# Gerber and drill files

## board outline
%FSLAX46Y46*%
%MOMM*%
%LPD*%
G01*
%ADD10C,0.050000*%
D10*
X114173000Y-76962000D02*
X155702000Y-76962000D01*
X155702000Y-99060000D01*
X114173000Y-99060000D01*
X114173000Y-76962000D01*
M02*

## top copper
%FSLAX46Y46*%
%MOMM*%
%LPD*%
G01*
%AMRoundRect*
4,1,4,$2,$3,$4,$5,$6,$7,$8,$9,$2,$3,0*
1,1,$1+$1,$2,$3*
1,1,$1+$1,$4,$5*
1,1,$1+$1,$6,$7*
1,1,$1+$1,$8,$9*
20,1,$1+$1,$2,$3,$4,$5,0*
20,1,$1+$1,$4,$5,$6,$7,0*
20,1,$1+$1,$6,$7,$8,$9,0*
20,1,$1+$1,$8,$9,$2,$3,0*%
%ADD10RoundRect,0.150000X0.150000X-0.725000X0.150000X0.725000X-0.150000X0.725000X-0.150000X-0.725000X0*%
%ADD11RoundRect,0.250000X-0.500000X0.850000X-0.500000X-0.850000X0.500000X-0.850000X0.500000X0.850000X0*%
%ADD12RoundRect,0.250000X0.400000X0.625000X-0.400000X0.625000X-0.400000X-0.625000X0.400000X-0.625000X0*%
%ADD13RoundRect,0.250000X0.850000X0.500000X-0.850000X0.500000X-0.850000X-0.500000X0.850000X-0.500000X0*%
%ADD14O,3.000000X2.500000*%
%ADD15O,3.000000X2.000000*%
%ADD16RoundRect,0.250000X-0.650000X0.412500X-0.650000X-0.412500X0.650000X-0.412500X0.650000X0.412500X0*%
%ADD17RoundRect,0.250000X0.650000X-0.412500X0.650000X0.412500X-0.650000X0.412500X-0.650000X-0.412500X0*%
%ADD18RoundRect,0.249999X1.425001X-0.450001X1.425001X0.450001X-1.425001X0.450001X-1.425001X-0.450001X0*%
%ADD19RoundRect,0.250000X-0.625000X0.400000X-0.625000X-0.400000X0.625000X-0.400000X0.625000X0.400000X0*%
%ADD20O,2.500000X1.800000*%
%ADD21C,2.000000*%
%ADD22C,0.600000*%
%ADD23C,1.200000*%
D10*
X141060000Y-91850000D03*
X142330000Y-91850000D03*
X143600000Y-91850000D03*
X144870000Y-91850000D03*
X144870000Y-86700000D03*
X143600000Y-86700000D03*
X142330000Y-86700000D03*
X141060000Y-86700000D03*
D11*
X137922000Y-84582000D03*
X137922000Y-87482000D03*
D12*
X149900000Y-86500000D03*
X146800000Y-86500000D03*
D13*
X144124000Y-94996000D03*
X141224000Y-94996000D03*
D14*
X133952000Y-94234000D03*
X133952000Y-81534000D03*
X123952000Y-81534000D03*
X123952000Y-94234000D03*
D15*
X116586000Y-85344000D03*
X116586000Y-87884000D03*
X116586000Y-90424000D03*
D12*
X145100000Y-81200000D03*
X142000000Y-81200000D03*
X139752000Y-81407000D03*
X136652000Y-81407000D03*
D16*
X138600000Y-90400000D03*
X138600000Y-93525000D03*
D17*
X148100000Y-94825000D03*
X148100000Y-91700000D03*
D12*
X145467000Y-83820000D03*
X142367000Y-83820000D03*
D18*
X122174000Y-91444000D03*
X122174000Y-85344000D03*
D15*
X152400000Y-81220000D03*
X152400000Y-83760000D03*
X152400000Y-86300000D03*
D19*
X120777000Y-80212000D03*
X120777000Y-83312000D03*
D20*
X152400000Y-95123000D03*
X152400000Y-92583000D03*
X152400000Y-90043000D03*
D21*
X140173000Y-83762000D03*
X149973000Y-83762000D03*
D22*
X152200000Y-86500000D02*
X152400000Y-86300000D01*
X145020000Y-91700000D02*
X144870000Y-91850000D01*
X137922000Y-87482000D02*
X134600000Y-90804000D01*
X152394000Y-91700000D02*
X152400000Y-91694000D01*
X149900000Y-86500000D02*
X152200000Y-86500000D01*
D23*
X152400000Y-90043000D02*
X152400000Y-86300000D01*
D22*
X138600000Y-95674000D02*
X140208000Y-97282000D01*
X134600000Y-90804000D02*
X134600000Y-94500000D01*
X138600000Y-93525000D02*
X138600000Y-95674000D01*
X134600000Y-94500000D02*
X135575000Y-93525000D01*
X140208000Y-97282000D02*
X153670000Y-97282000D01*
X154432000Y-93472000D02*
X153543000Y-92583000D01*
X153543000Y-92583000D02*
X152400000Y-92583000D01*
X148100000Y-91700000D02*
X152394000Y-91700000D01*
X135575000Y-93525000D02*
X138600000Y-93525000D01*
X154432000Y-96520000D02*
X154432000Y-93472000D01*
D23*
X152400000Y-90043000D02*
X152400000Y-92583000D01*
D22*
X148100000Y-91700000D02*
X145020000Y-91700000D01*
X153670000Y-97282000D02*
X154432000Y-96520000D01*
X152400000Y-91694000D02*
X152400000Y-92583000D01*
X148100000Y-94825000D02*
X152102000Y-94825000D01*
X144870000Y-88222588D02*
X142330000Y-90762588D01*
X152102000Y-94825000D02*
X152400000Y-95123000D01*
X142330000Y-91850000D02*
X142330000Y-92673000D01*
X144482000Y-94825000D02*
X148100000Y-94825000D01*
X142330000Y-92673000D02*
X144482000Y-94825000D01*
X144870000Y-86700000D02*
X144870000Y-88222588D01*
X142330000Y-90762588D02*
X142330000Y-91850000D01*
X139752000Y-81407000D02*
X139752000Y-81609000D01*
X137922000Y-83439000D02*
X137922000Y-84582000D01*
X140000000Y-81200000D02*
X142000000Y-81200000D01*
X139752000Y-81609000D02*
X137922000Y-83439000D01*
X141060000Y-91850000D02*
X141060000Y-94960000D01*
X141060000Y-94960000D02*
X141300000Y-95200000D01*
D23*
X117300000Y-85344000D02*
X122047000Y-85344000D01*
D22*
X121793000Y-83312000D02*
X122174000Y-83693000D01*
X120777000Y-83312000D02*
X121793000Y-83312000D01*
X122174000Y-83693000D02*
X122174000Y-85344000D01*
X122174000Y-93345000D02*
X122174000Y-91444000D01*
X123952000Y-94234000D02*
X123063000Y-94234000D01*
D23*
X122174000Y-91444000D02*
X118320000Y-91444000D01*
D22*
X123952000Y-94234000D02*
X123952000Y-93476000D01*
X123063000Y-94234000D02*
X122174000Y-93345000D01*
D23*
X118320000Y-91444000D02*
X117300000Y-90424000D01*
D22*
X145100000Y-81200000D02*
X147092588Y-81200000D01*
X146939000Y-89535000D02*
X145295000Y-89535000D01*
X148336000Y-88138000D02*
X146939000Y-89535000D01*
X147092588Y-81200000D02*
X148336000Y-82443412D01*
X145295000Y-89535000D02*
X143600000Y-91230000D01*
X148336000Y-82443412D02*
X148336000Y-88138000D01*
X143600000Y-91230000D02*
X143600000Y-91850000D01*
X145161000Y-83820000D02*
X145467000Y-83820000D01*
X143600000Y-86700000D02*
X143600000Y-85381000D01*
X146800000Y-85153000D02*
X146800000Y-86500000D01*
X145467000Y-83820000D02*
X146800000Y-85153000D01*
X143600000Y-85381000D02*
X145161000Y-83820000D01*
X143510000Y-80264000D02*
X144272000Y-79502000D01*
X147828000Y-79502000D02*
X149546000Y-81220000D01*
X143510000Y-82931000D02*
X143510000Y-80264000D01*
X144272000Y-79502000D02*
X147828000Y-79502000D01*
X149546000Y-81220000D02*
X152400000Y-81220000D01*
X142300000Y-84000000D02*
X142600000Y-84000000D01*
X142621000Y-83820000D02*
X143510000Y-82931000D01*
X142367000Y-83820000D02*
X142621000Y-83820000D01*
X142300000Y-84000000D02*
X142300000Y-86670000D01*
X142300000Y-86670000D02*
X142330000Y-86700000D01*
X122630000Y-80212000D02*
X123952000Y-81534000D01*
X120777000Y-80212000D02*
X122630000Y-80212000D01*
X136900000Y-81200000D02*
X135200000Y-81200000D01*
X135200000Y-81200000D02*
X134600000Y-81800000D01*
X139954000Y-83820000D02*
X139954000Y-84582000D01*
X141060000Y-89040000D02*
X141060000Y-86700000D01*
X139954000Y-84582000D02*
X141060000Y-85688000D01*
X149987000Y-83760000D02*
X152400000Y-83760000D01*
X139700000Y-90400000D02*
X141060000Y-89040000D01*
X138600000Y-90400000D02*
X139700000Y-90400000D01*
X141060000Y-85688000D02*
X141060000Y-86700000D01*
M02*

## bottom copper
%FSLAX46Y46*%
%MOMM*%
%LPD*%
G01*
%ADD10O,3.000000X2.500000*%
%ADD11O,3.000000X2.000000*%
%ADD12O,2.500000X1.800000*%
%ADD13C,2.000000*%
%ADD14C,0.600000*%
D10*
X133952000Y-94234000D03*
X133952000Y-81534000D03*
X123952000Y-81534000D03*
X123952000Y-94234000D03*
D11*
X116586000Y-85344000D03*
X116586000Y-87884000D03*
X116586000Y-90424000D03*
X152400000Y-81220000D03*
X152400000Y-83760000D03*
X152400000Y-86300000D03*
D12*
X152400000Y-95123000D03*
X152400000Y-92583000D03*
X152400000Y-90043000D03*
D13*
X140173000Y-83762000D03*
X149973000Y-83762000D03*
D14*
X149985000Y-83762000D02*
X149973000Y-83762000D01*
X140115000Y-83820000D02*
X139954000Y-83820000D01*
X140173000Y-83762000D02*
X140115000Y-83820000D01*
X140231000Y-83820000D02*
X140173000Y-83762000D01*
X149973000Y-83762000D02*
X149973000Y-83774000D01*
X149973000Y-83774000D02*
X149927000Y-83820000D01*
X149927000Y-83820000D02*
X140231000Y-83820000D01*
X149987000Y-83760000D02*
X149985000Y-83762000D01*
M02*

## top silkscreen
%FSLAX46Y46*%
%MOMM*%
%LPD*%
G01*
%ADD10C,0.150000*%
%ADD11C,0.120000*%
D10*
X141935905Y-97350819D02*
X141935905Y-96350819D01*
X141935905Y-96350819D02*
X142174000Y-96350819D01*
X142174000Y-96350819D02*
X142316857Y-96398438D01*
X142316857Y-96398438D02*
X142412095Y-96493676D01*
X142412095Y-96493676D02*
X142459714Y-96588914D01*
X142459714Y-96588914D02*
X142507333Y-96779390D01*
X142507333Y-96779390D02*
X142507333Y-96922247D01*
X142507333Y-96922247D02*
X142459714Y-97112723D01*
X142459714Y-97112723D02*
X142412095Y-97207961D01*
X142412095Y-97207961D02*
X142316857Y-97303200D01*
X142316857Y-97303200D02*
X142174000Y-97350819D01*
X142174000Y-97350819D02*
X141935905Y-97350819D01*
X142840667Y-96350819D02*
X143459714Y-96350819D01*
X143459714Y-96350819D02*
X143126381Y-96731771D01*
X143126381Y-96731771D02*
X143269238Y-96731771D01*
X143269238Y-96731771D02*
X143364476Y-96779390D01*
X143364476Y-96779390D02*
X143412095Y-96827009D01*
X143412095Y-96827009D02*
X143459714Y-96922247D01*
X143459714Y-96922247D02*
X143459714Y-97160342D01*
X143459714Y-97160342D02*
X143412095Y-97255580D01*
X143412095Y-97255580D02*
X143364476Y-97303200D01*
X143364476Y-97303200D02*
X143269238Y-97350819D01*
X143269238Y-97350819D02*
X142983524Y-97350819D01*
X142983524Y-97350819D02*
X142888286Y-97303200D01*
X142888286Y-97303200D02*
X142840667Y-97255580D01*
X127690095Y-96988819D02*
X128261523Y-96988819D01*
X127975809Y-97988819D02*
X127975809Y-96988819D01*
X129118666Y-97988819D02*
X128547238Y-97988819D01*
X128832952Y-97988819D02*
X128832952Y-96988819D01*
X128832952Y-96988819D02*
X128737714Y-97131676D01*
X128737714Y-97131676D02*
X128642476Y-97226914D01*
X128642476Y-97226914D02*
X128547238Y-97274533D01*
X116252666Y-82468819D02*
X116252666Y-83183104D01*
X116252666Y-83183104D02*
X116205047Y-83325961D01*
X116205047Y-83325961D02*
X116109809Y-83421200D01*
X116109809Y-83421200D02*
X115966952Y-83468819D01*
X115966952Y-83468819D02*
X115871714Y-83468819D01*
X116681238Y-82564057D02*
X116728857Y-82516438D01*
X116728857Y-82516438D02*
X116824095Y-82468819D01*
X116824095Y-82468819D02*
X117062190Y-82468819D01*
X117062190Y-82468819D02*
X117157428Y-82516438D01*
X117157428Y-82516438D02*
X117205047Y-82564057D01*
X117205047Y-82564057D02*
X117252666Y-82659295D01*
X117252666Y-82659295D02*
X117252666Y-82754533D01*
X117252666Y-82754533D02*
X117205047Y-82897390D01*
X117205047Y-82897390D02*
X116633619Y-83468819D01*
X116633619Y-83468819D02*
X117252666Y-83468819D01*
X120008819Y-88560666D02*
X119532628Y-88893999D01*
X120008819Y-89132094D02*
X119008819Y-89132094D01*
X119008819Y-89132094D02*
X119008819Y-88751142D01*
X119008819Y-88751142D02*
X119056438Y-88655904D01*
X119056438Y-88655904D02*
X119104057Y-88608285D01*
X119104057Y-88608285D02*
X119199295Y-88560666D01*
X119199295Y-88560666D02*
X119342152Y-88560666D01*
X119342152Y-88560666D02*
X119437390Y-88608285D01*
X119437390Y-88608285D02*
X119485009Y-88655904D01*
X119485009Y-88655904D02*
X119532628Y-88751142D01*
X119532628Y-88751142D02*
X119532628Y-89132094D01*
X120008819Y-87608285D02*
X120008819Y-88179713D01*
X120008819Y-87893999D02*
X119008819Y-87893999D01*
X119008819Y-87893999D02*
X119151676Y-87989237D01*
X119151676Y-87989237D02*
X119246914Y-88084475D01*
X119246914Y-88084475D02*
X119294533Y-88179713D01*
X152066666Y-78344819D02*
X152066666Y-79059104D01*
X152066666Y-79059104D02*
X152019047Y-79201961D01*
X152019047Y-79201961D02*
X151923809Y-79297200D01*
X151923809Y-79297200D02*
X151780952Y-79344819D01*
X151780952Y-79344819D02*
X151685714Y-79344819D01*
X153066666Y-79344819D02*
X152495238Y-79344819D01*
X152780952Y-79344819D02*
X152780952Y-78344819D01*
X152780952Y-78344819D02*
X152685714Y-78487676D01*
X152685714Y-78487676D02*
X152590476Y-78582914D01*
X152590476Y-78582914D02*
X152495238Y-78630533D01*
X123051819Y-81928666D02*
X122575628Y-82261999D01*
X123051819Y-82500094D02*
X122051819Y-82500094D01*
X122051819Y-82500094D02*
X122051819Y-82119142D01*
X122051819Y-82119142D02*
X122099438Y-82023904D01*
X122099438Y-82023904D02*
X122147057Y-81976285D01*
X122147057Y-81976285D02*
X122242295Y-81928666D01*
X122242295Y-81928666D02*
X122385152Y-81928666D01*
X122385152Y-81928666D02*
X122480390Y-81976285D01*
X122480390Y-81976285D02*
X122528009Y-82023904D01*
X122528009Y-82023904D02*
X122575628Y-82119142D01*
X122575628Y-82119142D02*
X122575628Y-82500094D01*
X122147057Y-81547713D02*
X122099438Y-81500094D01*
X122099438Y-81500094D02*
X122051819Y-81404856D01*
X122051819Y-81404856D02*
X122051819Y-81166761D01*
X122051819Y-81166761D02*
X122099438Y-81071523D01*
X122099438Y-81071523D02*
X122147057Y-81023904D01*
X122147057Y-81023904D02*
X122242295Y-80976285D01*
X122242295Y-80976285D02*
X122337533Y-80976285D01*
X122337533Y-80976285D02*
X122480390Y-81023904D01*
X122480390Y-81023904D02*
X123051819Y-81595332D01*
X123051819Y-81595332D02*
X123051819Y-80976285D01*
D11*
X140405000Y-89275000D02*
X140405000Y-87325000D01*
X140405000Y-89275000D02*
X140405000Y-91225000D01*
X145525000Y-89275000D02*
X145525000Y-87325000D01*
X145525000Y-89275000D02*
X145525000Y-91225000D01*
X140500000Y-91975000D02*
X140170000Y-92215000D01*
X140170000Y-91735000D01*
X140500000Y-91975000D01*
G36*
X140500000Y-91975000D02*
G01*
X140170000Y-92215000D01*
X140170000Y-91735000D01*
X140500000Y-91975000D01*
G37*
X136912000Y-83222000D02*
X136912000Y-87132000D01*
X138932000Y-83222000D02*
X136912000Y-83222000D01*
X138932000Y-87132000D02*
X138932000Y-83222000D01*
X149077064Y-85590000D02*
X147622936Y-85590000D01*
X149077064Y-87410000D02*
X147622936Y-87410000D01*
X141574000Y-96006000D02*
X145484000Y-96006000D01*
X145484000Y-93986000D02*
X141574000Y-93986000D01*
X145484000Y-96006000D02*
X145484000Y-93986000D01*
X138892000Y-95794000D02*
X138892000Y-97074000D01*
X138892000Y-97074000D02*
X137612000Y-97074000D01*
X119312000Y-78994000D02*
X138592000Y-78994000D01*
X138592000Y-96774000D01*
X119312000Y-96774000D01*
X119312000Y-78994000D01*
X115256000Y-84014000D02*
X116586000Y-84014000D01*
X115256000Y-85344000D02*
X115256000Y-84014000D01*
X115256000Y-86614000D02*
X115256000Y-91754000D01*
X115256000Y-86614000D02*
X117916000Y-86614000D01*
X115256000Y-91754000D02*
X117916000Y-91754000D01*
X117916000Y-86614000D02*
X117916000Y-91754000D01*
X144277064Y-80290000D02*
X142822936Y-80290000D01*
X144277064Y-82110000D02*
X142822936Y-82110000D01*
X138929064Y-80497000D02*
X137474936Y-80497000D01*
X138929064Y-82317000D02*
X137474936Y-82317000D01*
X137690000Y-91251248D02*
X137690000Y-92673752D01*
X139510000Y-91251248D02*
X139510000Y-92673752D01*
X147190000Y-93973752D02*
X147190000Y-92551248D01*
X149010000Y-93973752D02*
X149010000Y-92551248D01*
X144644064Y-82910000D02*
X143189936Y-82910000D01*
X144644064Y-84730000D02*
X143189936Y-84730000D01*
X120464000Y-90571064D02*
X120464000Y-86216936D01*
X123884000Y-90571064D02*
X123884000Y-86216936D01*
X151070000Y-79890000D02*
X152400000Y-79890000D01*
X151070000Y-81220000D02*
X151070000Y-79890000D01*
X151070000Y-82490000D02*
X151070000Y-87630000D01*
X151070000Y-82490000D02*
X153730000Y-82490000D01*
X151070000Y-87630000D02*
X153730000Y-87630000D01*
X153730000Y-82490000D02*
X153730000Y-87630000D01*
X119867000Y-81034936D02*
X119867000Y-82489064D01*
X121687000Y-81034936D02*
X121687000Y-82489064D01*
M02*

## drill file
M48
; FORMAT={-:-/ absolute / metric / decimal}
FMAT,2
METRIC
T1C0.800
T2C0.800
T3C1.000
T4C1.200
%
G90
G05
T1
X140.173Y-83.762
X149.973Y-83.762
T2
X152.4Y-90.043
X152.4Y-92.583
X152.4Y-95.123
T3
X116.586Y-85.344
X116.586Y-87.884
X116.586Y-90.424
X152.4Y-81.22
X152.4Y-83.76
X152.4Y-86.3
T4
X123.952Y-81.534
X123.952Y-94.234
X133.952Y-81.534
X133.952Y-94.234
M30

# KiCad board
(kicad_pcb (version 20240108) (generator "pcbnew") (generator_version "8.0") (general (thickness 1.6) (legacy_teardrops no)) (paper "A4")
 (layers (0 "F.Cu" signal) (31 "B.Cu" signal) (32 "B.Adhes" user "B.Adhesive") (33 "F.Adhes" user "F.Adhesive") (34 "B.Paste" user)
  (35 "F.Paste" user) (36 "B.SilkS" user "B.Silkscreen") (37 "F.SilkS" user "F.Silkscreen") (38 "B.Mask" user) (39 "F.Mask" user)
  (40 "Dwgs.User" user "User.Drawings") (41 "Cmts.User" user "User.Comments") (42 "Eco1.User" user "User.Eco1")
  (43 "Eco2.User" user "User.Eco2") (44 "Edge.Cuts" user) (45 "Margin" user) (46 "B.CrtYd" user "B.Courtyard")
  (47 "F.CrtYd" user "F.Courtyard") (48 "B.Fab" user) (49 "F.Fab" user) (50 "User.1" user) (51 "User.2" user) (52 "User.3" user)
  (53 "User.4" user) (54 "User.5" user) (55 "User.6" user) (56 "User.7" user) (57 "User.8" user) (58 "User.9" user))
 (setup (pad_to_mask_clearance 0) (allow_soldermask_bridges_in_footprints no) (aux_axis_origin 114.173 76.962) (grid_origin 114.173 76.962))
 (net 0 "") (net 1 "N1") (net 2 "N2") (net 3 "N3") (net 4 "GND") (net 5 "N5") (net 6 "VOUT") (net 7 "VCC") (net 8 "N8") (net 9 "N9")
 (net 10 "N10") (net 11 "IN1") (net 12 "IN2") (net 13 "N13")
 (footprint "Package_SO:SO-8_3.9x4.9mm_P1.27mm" (layer "F.Cu") (at 142.965 89.275 90)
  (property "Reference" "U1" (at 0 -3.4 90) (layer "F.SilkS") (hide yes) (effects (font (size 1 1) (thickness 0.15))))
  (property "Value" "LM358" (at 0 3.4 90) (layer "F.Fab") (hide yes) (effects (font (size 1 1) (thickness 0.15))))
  (fp_line (start 0 -2.56) (end 1.95 -2.56) (stroke (width 0.12) (type solid)) (layer "F.SilkS"))
  (fp_line (start 0 -2.56) (end -1.95 -2.56) (stroke (width 0.12) (type solid)) (layer "F.SilkS"))
  (fp_line (start 0 2.56) (end 1.95 2.56) (stroke (width 0.12) (type solid)) (layer "F.SilkS"))
  (fp_line (start 0 2.56) (end -1.95 2.56) (stroke (width 0.12) (type solid)) (layer "F.SilkS"))
  (fp_poly
   (pts (xy -2.7 -2.465) (xy -2.94 -2.795) (xy -2.46 -2.795) (xy -2.7 -2.465)) (stroke (width 0.12) (type solid)) (fill solid)
   (layer "F.SilkS"))
  (pad "1" smd roundrect (at -2.575 -1.905 90) (size 1.75 0.6) (layers "F.Cu" "F.Paste" "F.Mask") (roundrect_rratio 0.25) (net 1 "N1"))
  (pad "2" smd roundrect (at -2.575 -0.635 90) (size 1.75 0.6) (layers "F.Cu" "F.Paste" "F.Mask") (roundrect_rratio 0.25) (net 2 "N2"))
  (pad "3" smd roundrect (at -2.575 0.635 90) (size 1.75 0.6) (layers "F.Cu" "F.Paste" "F.Mask") (roundrect_rratio 0.25) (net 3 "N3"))
  (pad "4" smd roundrect (at -2.575 1.905 90) (size 1.75 0.6) (layers "F.Cu" "F.Paste" "F.Mask") (roundrect_rratio 0.25) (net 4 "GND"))
  (pad "5" smd roundrect (at 2.575 1.905 90) (size 1.75 0.6) (layers "F.Cu" "F.Paste" "F.Mask") (roundrect_rratio 0.25) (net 2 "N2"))
  (pad "6" smd roundrect (at 2.575 0.635 90) (size 1.75 0.6) (layers "F.Cu" "F.Paste" "F.Mask") (roundrect_rratio 0.25) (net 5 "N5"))
  (pad "7" smd roundrect (at 2.575 -0.635 90) (size 1.75 0.6) (layers "F.Cu" "F.Paste" "F.Mask") (roundrect_rratio 0.25) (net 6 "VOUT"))
  (pad "8" smd roundrect (at 2.575 -1.905 90) (size 1.75 0.6) (layers "F.Cu" "F.Paste" "F.Mask") (roundrect_rratio 0.25) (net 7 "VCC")))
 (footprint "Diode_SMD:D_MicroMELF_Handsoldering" (layer "F.Cu") (at 137.922 86.032 -90)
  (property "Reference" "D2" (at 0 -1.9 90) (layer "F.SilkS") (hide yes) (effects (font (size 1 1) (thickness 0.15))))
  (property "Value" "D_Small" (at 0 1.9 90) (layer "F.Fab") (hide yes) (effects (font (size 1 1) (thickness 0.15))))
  (fp_line (start -2.81 1.01) (end 1.1 1.01) (stroke (width 0.12) (type solid)) (layer "F.SilkS"))
  (fp_line (start -2.81 -1.01) (end -2.81 1.01) (stroke (width 0.12) (type solid)) (layer "F.SilkS"))
  (fp_line (start 1.1 -1.01) (end -2.81 -1.01) (stroke (width 0.12) (type solid)) (layer "F.SilkS"))
  (pad "1" smd roundrect (at -1.45 0 270) (size 2.2 1.5) (layers "F.Cu" "F.Paste" "F.Mask") (roundrect_rratio 0.1666666667) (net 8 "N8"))
  (pad "2" smd roundrect (at 1.45 0 270) (size 2.2 1.5) (layers "F.Cu" "F.Paste" "F.Mask") (roundrect_rratio 0.1666666667) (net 4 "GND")))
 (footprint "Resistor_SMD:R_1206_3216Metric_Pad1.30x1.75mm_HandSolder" (layer "F.Cu") (at 148.35 86.5 180)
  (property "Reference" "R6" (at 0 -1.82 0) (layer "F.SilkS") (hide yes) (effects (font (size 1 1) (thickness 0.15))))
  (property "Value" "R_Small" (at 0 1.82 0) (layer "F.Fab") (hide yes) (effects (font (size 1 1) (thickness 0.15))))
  (fp_line (start -0.727064 0.91) (end 0.727064 0.91) (stroke (width 0.12) (type solid)) (layer "F.SilkS"))
  (fp_line (start -0.727064 -0.91) (end 0.727064 -0.91) (stroke (width 0.12) (type solid)) (layer "F.SilkS"))
  (pad "1" smd roundrect (at -1.55 0 180) (size 1.3 1.75) (layers "F.Cu" "F.Paste" "F.Mask") (roundrect_rratio 0.192308) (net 4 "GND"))
  (pad "2" smd roundrect (at 1.55 0 180) (size 1.3 1.75) (layers "F.Cu" "F.Paste" "F.Mask") (roundrect_rratio 0.192308) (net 5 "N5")))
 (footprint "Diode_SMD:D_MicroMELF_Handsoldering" (layer "F.Cu") (at 142.674 94.996 180)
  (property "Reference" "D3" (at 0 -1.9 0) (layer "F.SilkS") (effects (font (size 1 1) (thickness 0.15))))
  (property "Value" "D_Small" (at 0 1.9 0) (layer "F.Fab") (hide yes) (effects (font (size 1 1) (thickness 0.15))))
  (fp_line (start 1.1 -1.01) (end -2.81 -1.01) (stroke (width 0.12) (type solid)) (layer "F.SilkS"))
  (fp_line (start -2.81 1.01) (end 1.1 1.01) (stroke (width 0.12) (type solid)) (layer "F.SilkS"))
  (fp_line (start -2.81 -1.01) (end -2.81 1.01) (stroke (width 0.12) (type solid)) (layer "F.SilkS"))
  (pad "1" smd roundrect (at -1.45 0 180) (size 2.2 1.5) (layers "F.Cu" "F.Paste" "F.Mask") (roundrect_rratio 0.1666666667) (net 2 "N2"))
  (pad "2" smd roundrect (at 1.45 0 180) (size 2.2 1.5) (layers "F.Cu" "F.Paste" "F.Mask") (roundrect_rratio 0.1666666667) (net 1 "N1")))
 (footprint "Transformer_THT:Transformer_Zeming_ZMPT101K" (layer "F.Cu") (at 133.952 94.234 180)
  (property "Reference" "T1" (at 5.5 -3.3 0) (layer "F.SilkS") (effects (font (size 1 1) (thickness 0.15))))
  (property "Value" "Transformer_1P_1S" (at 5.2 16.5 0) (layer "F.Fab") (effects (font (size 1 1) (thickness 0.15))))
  (fp_line (start -4.94 -1.56) (end -4.94 -2.84) (stroke (width 0.12) (type default)) (layer "F.SilkS"))
  (fp_line (start -4.94 -2.84) (end -3.66 -2.84) (stroke (width 0.12) (type default)) (layer "F.SilkS"))
  (fp_rect (start -4.64 -2.54) (end 14.64 15.24) (stroke (width 0.12) (type default)) (fill none) (layer "F.SilkS"))
  (pad "1" thru_hole oval (at 0 0 180) (size 3 2.5) (drill 1.2) (layers "*.Cu" "*.Mask") (remove_unused_layers no) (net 4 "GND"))
  (pad "2" thru_hole oval (at 0 12.7 180) (size 3 2.5) (drill 1.2) (layers "*.Cu" "*.Mask") (remove_unused_layers no) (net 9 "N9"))
  (pad "3" thru_hole oval (at 10 12.7 180) (size 3 2.5) (drill 1.2) (layers "*.Cu" "*.Mask") (remove_unused_layers no) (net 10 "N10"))
  (pad "4" thru_hole oval (at 10 0 180) (size 3 2.5) (drill 1.2) (layers "*.Cu" "*.Mask") (remove_unused_layers no) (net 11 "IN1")))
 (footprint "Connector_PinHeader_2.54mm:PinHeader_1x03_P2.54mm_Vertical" (layer "F.Cu") (at 116.586 85.344)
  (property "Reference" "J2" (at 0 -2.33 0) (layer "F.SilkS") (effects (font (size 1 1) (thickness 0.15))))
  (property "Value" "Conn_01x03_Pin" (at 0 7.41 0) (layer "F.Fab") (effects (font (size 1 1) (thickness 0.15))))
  (fp_line (start -1.33 -1.33) (end 0 -1.33) (stroke (width 0.12) (type solid)) (layer "F.SilkS"))
  (fp_line (start -1.33 0) (end -1.33 -1.33) (stroke (width 0.12) (type solid)) (layer "F.SilkS"))
  (fp_line (start -1.33 1.27) (end -1.33 6.41) (stroke (width 0.12) (type solid)) (layer "F.SilkS"))
  (fp_line (start -1.33 1.27) (end 1.33 1.27) (stroke (width 0.12) (type solid)) (layer "F.SilkS"))
  (fp_line (start -1.33 6.41) (end 1.33 6.41) (stroke (width 0.12) (type solid)) (layer "F.SilkS"))
  (fp_line (start 1.33 1.27) (end 1.33 6.41) (stroke (width 0.12) (type solid)) (layer "F.SilkS"))
  (pad "1" thru_hole oval (at 0 0) (size 3 2) (drill 1) (layers "*.Cu" "*.Mask") (remove_unused_layers no) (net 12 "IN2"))
  (pad "2" thru_hole oval (at 0 2.54) (size 3 2) (drill 1) (layers "*.Cu" "*.Mask") (remove_unused_layers no) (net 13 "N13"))
  (pad "3" thru_hole oval (at 0 5.08) (size 3 2) (drill 1) (layers "*.Cu" "*.Mask") (remove_unused_layers no) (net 11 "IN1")))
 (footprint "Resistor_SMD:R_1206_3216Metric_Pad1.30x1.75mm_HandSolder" (layer "F.Cu") (at 143.55 81.2 180)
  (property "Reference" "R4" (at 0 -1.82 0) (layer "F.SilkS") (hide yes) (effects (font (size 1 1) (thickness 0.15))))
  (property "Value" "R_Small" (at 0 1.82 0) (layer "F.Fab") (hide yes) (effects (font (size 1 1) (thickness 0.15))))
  (fp_line (start -0.727064 0.91) (end 0.727064 0.91) (stroke (width 0.12) (type solid)) (layer "F.SilkS"))
  (fp_line (start -0.727064 -0.91) (end 0.727064 -0.91) (stroke (width 0.12) (type solid)) (layer "F.SilkS"))
  (pad "1" smd roundrect (at -1.55 0 180) (size 1.3 1.75) (layers "F.Cu" "F.Paste" "F.Mask") (roundrect_rratio 0.192308) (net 3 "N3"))
  (pad "2" smd roundrect (at 1.55 0 180) (size 1.3 1.75) (layers "F.Cu" "F.Paste" "F.Mask") (roundrect_rratio 0.192308) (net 8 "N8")))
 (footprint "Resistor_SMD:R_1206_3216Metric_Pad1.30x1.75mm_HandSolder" (layer "F.Cu") (at 138.202 81.407 180)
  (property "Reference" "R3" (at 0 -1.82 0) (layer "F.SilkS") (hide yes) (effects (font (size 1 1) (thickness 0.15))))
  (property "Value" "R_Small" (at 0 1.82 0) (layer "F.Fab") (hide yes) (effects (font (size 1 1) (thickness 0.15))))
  (fp_line (start -0.727064 0.91) (end 0.727064 0.91) (stroke (width 0.12) (type solid)) (layer "F.SilkS"))
  (fp_line (start -0.727064 -0.91) (end 0.727064 -0.91) (stroke (width 0.12) (type solid)) (layer "F.SilkS"))
  (pad "1" smd roundrect (at -1.55 0 180) (size 1.3 1.75) (layers "F.Cu" "F.Paste" "F.Mask") (roundrect_rratio 0.192308) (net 8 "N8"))
  (pad "2" smd roundrect (at 1.55 0 180) (size 1.3 1.75) (layers "F.Cu" "F.Paste" "F.Mask") (roundrect_rratio 0.192308) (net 9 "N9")))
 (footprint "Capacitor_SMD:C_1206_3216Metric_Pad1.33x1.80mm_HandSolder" (layer "F.Cu") (at 138.6 91.9625 -90)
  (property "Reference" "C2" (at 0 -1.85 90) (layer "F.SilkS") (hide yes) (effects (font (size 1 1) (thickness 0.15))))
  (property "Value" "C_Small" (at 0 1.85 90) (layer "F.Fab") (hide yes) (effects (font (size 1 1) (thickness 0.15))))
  (fp_line (start -0.711252 0.91) (end 0.711252 0.91) (stroke (width 0.12) (type solid)) (layer "F.SilkS"))
  (fp_line (start -0.711252 -0.91) (end 0.711252 -0.91) (stroke (width 0.12) (type solid)) (layer "F.SilkS"))
  (pad "1" smd roundrect (at -1.5625 0 270) (size 1.325 1.8) (layers "F.Cu" "F.Paste" "F.Mask") (roundrect_rratio 0.188679) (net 7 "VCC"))
  (pad "2" smd roundrect (at 1.5625 0 270) (size 1.325 1.8) (layers "F.Cu" "F.Paste" "F.Mask") (roundrect_rratio 0.188679) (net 4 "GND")))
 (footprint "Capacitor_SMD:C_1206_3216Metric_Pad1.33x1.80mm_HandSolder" (layer "F.Cu") (at 148.1 93.2625 90)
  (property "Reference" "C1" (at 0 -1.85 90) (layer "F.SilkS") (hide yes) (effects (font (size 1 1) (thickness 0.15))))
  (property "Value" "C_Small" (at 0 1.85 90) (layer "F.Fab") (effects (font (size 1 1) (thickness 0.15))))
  (fp_line (start -0.711252 -0.91) (end 0.711252 -0.91) (stroke (width 0.12) (type solid)) (layer "F.SilkS"))
  (fp_line (start -0.711252 0.91) (end 0.711252 0.91) (stroke (width 0.12) (type solid)) (layer "F.SilkS"))
  (pad "1" smd roundrect (at -1.5625 0 90) (size 1.325 1.8) (layers "F.Cu" "F.Paste" "F.Mask") (roundrect_rratio 0.188679) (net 2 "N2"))
  (pad "2" smd roundrect (at 1.5625 0 90) (size 1.325 1.8) (layers "F.Cu" "F.Paste" "F.Mask") (roundrect_rratio 0.188679) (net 4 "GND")))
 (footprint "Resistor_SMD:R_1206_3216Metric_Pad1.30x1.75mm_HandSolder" (layer "F.Cu") (at 143.917 83.82 180)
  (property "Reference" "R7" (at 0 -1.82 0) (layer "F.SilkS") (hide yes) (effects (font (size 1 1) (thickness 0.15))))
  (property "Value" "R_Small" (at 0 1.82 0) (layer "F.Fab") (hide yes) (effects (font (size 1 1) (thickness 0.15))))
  (fp_line (start -0.727064 0.91) (end 0.727064 0.91) (stroke (width 0.12) (type solid)) (layer "F.SilkS"))
  (fp_line (start -0.727064 -0.91) (end 0.727064 -0.91) (stroke (width 0.12) (type solid)) (layer "F.SilkS"))
  (pad "1" smd roundrect (at -1.55 0 180) (size 1.3 1.75) (layers "F.Cu" "F.Paste" "F.Mask") (roundrect_rratio 0.192308) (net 5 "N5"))
  (pad "2" smd roundrect (at 1.55 0 180) (size 1.3 1.75) (layers "F.Cu" "F.Paste" "F.Mask") (roundrect_rratio 0.192308) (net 6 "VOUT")))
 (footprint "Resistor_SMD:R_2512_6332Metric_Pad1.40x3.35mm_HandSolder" (layer "F.Cu") (at 122.174 88.394 90)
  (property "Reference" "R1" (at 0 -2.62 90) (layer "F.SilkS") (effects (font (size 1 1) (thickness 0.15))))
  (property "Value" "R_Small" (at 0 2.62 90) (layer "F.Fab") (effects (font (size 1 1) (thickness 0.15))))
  (fp_line (start -2.177064 -1.71) (end 2.177064 -1.71) (stroke (width 0.12) (type solid)) (layer "F.SilkS"))
  (fp_line (start -2.177064 1.71) (end 2.177064 1.71) (stroke (width 0.12) (type solid)) (layer "F.SilkS"))
  (pad "1" smd roundrect (at -3.05 0 90) (size 1.4 3.35) (layers "F.Cu" "F.Paste" "F.Mask") (roundrect_rratio 0.178571) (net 11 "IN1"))
  (pad "2" smd roundrect (at 3.05 0 90) (size 1.4 3.35) (layers "F.Cu" "F.Paste" "F.Mask") (roundrect_rratio 0.178571) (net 12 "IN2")))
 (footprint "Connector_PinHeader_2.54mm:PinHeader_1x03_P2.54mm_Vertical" (layer "F.Cu") (at 152.4 81.22)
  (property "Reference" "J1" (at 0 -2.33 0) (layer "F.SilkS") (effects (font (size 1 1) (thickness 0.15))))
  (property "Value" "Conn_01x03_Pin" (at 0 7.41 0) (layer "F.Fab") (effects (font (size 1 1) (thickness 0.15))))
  (fp_line (start -1.33 -1.33) (end 0 -1.33) (stroke (width 0.12) (type solid)) (layer "F.SilkS"))
  (fp_line (start -1.33 0) (end -1.33 -1.33) (stroke (width 0.12) (type solid)) (layer "F.SilkS"))
  (fp_line (start -1.33 1.27) (end -1.33 6.41) (stroke (width 0.12) (type solid)) (layer "F.SilkS"))
  (fp_line (start -1.33 1.27) (end 1.33 1.27) (stroke (width 0.12) (type solid)) (layer "F.SilkS"))
  (fp_line (start -1.33 6.41) (end 1.33 6.41) (stroke (width 0.12) (type solid)) (layer "F.SilkS"))
  (fp_line (start 1.33 1.27) (end 1.33 6.41) (stroke (width 0.12) (type solid)) (layer "F.SilkS"))
  (pad "1" thru_hole oval (at 0 0) (size 3 2) (drill 1) (layers "*.Cu" "*.Mask") (remove_unused_layers no) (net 6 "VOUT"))
  (pad "2" thru_hole oval (at 0 2.54) (size 3 2) (drill 1) (layers "*.Cu" "*.Mask") (remove_unused_layers no) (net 7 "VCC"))
  (pad "3" thru_hole oval (at 0 5.08) (size 3 2) (drill 1) (layers "*.Cu" "*.Mask") (remove_unused_layers no) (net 4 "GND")))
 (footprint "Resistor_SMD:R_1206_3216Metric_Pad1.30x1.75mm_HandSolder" (layer "F.Cu") (at 120.777 81.762 -90)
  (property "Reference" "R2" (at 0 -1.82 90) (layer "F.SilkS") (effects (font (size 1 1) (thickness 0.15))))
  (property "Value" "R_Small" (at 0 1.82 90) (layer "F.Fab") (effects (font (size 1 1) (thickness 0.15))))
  (fp_line (start -0.727064 0.91) (end 0.727064 0.91) (stroke (width 0.12) (type solid)) (layer "F.SilkS"))
  (fp_line (start -0.727064 -0.91) (end 0.727064 -0.91) (stroke (width 0.12) (type solid)) (layer "F.SilkS"))
  (pad "1" smd roundrect (at -1.55 0 270) (size 1.3 1.75) (layers "F.Cu" "F.Paste" "F.Mask") (roundrect_rratio 0.192308) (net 10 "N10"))
  (pad "2" smd roundrect (at 1.55 0 270) (size 1.3 1.75) (layers "F.Cu" "F.Paste" "F.Mask") (roundrect_rratio 0.192308) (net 12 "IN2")))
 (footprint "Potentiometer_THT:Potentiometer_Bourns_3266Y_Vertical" (layer "B.Cu") (at 152.4 95.123 -90)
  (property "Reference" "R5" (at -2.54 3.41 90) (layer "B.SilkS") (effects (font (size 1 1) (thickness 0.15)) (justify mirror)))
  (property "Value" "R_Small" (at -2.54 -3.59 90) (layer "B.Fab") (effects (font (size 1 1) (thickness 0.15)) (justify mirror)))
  (pad "1" thru_hole oval (at 0 0 270) (size 1.8 2.5) (drill 0.8) (layers "*.Cu" "*.Mask") (remove_unused_layers no) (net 2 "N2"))
  (pad "2" thru_hole oval (at -2.54 0 270) (size 1.8 2.5) (drill 0.8) (layers "*.Cu" "*.Mask") (remove_unused_layers no) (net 4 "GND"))
  (pad "3" thru_hole oval (at -5.08 0 270) (size 1.8 2.5) (drill 0.8) (layers "*.Cu" "*.Mask") (remove_unused_layers no) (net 4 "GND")))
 (gr_rect (start 114.173 76.962) (end 155.702 99.06) (stroke (width 0.05) (type default)) (fill none) (layer "Edge.Cuts"))
 (segment (start 152.2 86.5) (end 152.4 86.3) (width 0.6) (layer "F.Cu") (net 4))
 (segment (start 145.02 91.7) (end 144.87 91.85) (width 0.6) (layer "F.Cu") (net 4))
 (segment (start 137.922 87.482) (end 134.6 90.804) (width 0.6) (layer "F.Cu") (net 4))
 (segment (start 152.394 91.7) (end 152.4 91.694) (width 0.6) (layer "F.Cu") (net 4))
 (segment (start 149.9 86.5) (end 152.2 86.5) (width 0.6) (layer "F.Cu") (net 4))
 (segment (start 152.4 90.043) (end 152.4 86.3) (width 1.2) (layer "F.Cu") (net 4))
 (segment (start 138.6 95.674) (end 140.208 97.282) (width 0.6) (layer "F.Cu") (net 4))
 (segment (start 134.6 90.804) (end 134.6 94.5) (width 0.6) (layer "F.Cu") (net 4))
 (segment (start 138.6 93.525) (end 138.6 95.674) (width 0.6) (layer "F.Cu") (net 4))
 (segment (start 134.6 94.5) (end 135.575 93.525) (width 0.6) (layer "F.Cu") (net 4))
 (segment (start 140.208 97.282) (end 153.67 97.282) (width 0.6) (layer "F.Cu") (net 4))
 (segment (start 154.432 93.472) (end 153.543 92.583) (width 0.6) (layer "F.Cu") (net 4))
 (segment (start 153.543 92.583) (end 152.4 92.583) (width 0.6) (layer "F.Cu") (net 4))
 (segment (start 148.1 91.7) (end 152.394 91.7) (width 0.6) (layer "F.Cu") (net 4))
 (segment (start 135.575 93.525) (end 138.6 93.525) (width 0.6) (layer "F.Cu") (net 4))
 (segment (start 154.432 96.52) (end 154.432 93.472) (width 0.6) (layer "F.Cu") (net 4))
 (segment (start 152.4 90.043) (end 152.4 92.583) (width 1.2) (layer "F.Cu") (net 4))
 (segment (start 148.1 91.7) (end 145.02 91.7) (width 0.6) (layer "F.Cu") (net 4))
 (segment (start 153.67 97.282) (end 154.432 96.52) (width 0.6) (layer "F.Cu") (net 4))
 (segment (start 152.4 91.694) (end 152.4 92.583) (width 0.6) (layer "F.Cu") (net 4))
 (segment (start 148.1 94.825) (end 152.102 94.825) (width 0.6) (layer "F.Cu") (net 2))
 (segment (start 144.87 88.222588) (end 142.33 90.762588) (width 0.6) (layer "F.Cu") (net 2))
 (segment (start 152.102 94.825) (end 152.4 95.123) (width 0.6) (layer "F.Cu") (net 2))
 (segment (start 142.33 91.85) (end 142.33 92.673) (width 0.6) (layer "F.Cu") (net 2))
 (segment (start 144.482 94.825) (end 148.1 94.825) (width 0.6) (layer "F.Cu") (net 2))
 (segment (start 142.33 92.673) (end 144.482 94.825) (width 0.6) (layer "F.Cu") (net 2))
 (segment (start 144.87 86.7) (end 144.87 88.222588) (width 0.6) (layer "F.Cu") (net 2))
 (segment (start 142.33 90.762588) (end 142.33 91.85) (width 0.6) (layer "F.Cu") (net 2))
 (segment (start 139.752 81.407) (end 139.752 81.609) (width 0.6) (layer "F.Cu") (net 8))
 (segment (start 137.922 83.439) (end 137.922 84.582) (width 0.6) (layer "F.Cu") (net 8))
 (segment (start 140 81.2) (end 142 81.2) (width 0.6) (layer "F.Cu") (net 8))
 (segment (start 139.752 81.609) (end 137.922 83.439) (width 0.6) (layer "F.Cu") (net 8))
 (segment (start 141.06 91.85) (end 141.06 94.96) (width 0.6) (layer "F.Cu") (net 1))
 (segment (start 141.06 94.96) (end 141.3 95.2) (width 0.6) (layer "F.Cu") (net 1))
 (segment (start 117.3 85.344) (end 122.047 85.344) (width 1.2) (layer "F.Cu") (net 12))
 (segment (start 121.793 83.312) (end 122.174 83.693) (width 0.6) (layer "F.Cu") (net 12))
 (segment (start 120.777 83.312) (end 121.793 83.312) (width 0.6) (layer "F.Cu") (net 12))
 (segment (start 122.174 83.693) (end 122.174 85.344) (width 0.6) (layer "F.Cu") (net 12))
 (segment (start 122.174 93.345) (end 122.174 91.444) (width 0.6) (layer "F.Cu") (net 11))
 (segment (start 123.952 94.234) (end 123.063 94.234) (width 0.6) (layer "F.Cu") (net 11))
 (segment (start 122.174 91.444) (end 118.32 91.444) (width 1.2) (layer "F.Cu") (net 11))
 (segment (start 123.952 94.234) (end 123.952 93.476) (width 0.6) (layer "F.Cu") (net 11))
 (segment (start 123.063 94.234) (end 122.174 93.345) (width 0.6) (layer "F.Cu") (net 11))
 (segment (start 118.32 91.444) (end 117.3 90.424) (width 1.2) (layer "F.Cu") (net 11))
 (segment (start 145.1 81.2) (end 147.092588 81.2) (width 0.6) (layer "F.Cu") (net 3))
 (segment (start 146.939 89.535) (end 145.295 89.535) (width 0.6) (layer "F.Cu") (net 3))
 (segment (start 148.336 88.138) (end 146.939 89.535) (width 0.6) (layer "F.Cu") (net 3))
 (segment (start 147.092588 81.2) (end 148.336 82.443412) (width 0.6) (layer "F.Cu") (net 3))
 (segment (start 145.295 89.535) (end 143.6 91.23) (width 0.6) (layer "F.Cu") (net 3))
 (segment (start 148.336 82.443412) (end 148.336 88.138) (width 0.6) (layer "F.Cu") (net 3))
 (segment (start 143.6 91.23) (end 143.6 91.85) (width 0.6) (layer "F.Cu") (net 3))
 (segment (start 145.161 83.82) (end 145.467 83.82) (width 0.6) (layer "F.Cu") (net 5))
 (segment (start 143.6 86.7) (end 143.6 85.381) (width 0.6) (layer "F.Cu") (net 5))
 (segment (start 146.8 85.153) (end 146.8 86.5) (width 0.6) (layer "F.Cu") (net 5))
 (segment (start 145.467 83.82) (end 146.8 85.153) (width 0.6) (layer "F.Cu") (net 5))
 (segment (start 143.6 85.381) (end 145.161 83.82) (width 0.6) (layer "F.Cu") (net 5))
 (segment (start 143.51 80.264) (end 144.272 79.502) (width 0.6) (layer "F.Cu") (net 6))
 (segment (start 147.828 79.502) (end 149.546 81.22) (width 0.6) (layer "F.Cu") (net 6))
 (segment (start 143.51 82.931) (end 143.51 80.264) (width 0.6) (layer "F.Cu") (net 6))
 (segment (start 144.272 79.502) (end 147.828 79.502) (width 0.6) (layer "F.Cu") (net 6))
 (segment (start 149.546 81.22) (end 152.4 81.22) (width 0.6) (layer "F.Cu") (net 6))
 (segment (start 142.3 84) (end 142.6 84) (width 0.6) (layer "F.Cu") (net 6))
 (segment (start 142.621 83.82) (end 143.51 82.931) (width 0.6) (layer "F.Cu") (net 6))
 (segment (start 142.367 83.82) (end 142.621 83.82) (width 0.6) (layer "F.Cu") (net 6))
 (segment (start 142.3 84) (end 142.3 86.67) (width 0.6) (layer "F.Cu") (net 6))
 (segment (start 142.3 86.67) (end 142.33 86.7) (width 0.6) (layer "F.Cu") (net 6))
 (segment (start 122.63 80.212) (end 123.952 81.534) (width 0.6) (layer "F.Cu") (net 10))
 (segment (start 120.777 80.212) (end 122.63 80.212) (width 0.6) (layer "F.Cu") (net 10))
 (segment (start 136.9 81.2) (end 135.2 81.2) (width 0.6) (layer "F.Cu") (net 9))
 (segment (start 135.2 81.2) (end 134.6 81.8) (width 0.6) (layer "F.Cu") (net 9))
 (segment (start 139.954 83.82) (end 139.954 84.582) (width 0.6) (layer "F.Cu") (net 7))
 (segment (start 141.06 89.04) (end 141.06 86.7) (width 0.6) (layer "F.Cu") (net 7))
 (segment (start 139.954 84.582) (end 141.06 85.688) (width 0.6) (layer "F.Cu") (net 7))
 (segment (start 149.987 83.76) (end 152.4 83.76) (width 0.6) (layer "F.Cu") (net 7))
 (segment (start 139.7 90.4) (end 141.06 89.04) (width 0.6) (layer "F.Cu") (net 7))
 (segment (start 138.6 90.4) (end 139.7 90.4) (width 0.6) (layer "F.Cu") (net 7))
 (segment (start 141.06 85.688) (end 141.06 86.7) (width 0.6) (layer "F.Cu") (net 7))
 (via (at 140.173 83.762) (size 2) (drill 0.8) (layers "F.Cu" "B.Cu") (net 7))
 (via (at 149.973 83.762) (size 2) (drill 0.8) (layers "F.Cu" "B.Cu") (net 7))
 (segment (start 149.985 83.762) (end 149.973 83.762) (width 0.6) (layer "B.Cu") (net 7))
 (segment (start 140.115 83.82) (end 139.954 83.82) (width 0.6) (layer "B.Cu") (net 7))
 (segment (start 140.173 83.762) (end 140.115 83.82) (width 0.6) (layer "B.Cu") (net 7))
 (segment (start 140.231 83.82) (end 140.173 83.762) (width 0.6) (layer "B.Cu") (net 7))
 (segment (start 149.973 83.762) (end 149.973 83.774) (width 0.6) (layer "B.Cu") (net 7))
 (segment (start 149.973 83.774) (end 149.927 83.82) (width 0.6) (layer "B.Cu") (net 7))
 (segment (start 149.927 83.82) (end 140.231 83.82) (width 0.6) (layer "B.Cu") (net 7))
 (segment (start 149.987 83.76) (end 149.985 83.762) (width 0.6) (layer "B.Cu") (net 7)))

